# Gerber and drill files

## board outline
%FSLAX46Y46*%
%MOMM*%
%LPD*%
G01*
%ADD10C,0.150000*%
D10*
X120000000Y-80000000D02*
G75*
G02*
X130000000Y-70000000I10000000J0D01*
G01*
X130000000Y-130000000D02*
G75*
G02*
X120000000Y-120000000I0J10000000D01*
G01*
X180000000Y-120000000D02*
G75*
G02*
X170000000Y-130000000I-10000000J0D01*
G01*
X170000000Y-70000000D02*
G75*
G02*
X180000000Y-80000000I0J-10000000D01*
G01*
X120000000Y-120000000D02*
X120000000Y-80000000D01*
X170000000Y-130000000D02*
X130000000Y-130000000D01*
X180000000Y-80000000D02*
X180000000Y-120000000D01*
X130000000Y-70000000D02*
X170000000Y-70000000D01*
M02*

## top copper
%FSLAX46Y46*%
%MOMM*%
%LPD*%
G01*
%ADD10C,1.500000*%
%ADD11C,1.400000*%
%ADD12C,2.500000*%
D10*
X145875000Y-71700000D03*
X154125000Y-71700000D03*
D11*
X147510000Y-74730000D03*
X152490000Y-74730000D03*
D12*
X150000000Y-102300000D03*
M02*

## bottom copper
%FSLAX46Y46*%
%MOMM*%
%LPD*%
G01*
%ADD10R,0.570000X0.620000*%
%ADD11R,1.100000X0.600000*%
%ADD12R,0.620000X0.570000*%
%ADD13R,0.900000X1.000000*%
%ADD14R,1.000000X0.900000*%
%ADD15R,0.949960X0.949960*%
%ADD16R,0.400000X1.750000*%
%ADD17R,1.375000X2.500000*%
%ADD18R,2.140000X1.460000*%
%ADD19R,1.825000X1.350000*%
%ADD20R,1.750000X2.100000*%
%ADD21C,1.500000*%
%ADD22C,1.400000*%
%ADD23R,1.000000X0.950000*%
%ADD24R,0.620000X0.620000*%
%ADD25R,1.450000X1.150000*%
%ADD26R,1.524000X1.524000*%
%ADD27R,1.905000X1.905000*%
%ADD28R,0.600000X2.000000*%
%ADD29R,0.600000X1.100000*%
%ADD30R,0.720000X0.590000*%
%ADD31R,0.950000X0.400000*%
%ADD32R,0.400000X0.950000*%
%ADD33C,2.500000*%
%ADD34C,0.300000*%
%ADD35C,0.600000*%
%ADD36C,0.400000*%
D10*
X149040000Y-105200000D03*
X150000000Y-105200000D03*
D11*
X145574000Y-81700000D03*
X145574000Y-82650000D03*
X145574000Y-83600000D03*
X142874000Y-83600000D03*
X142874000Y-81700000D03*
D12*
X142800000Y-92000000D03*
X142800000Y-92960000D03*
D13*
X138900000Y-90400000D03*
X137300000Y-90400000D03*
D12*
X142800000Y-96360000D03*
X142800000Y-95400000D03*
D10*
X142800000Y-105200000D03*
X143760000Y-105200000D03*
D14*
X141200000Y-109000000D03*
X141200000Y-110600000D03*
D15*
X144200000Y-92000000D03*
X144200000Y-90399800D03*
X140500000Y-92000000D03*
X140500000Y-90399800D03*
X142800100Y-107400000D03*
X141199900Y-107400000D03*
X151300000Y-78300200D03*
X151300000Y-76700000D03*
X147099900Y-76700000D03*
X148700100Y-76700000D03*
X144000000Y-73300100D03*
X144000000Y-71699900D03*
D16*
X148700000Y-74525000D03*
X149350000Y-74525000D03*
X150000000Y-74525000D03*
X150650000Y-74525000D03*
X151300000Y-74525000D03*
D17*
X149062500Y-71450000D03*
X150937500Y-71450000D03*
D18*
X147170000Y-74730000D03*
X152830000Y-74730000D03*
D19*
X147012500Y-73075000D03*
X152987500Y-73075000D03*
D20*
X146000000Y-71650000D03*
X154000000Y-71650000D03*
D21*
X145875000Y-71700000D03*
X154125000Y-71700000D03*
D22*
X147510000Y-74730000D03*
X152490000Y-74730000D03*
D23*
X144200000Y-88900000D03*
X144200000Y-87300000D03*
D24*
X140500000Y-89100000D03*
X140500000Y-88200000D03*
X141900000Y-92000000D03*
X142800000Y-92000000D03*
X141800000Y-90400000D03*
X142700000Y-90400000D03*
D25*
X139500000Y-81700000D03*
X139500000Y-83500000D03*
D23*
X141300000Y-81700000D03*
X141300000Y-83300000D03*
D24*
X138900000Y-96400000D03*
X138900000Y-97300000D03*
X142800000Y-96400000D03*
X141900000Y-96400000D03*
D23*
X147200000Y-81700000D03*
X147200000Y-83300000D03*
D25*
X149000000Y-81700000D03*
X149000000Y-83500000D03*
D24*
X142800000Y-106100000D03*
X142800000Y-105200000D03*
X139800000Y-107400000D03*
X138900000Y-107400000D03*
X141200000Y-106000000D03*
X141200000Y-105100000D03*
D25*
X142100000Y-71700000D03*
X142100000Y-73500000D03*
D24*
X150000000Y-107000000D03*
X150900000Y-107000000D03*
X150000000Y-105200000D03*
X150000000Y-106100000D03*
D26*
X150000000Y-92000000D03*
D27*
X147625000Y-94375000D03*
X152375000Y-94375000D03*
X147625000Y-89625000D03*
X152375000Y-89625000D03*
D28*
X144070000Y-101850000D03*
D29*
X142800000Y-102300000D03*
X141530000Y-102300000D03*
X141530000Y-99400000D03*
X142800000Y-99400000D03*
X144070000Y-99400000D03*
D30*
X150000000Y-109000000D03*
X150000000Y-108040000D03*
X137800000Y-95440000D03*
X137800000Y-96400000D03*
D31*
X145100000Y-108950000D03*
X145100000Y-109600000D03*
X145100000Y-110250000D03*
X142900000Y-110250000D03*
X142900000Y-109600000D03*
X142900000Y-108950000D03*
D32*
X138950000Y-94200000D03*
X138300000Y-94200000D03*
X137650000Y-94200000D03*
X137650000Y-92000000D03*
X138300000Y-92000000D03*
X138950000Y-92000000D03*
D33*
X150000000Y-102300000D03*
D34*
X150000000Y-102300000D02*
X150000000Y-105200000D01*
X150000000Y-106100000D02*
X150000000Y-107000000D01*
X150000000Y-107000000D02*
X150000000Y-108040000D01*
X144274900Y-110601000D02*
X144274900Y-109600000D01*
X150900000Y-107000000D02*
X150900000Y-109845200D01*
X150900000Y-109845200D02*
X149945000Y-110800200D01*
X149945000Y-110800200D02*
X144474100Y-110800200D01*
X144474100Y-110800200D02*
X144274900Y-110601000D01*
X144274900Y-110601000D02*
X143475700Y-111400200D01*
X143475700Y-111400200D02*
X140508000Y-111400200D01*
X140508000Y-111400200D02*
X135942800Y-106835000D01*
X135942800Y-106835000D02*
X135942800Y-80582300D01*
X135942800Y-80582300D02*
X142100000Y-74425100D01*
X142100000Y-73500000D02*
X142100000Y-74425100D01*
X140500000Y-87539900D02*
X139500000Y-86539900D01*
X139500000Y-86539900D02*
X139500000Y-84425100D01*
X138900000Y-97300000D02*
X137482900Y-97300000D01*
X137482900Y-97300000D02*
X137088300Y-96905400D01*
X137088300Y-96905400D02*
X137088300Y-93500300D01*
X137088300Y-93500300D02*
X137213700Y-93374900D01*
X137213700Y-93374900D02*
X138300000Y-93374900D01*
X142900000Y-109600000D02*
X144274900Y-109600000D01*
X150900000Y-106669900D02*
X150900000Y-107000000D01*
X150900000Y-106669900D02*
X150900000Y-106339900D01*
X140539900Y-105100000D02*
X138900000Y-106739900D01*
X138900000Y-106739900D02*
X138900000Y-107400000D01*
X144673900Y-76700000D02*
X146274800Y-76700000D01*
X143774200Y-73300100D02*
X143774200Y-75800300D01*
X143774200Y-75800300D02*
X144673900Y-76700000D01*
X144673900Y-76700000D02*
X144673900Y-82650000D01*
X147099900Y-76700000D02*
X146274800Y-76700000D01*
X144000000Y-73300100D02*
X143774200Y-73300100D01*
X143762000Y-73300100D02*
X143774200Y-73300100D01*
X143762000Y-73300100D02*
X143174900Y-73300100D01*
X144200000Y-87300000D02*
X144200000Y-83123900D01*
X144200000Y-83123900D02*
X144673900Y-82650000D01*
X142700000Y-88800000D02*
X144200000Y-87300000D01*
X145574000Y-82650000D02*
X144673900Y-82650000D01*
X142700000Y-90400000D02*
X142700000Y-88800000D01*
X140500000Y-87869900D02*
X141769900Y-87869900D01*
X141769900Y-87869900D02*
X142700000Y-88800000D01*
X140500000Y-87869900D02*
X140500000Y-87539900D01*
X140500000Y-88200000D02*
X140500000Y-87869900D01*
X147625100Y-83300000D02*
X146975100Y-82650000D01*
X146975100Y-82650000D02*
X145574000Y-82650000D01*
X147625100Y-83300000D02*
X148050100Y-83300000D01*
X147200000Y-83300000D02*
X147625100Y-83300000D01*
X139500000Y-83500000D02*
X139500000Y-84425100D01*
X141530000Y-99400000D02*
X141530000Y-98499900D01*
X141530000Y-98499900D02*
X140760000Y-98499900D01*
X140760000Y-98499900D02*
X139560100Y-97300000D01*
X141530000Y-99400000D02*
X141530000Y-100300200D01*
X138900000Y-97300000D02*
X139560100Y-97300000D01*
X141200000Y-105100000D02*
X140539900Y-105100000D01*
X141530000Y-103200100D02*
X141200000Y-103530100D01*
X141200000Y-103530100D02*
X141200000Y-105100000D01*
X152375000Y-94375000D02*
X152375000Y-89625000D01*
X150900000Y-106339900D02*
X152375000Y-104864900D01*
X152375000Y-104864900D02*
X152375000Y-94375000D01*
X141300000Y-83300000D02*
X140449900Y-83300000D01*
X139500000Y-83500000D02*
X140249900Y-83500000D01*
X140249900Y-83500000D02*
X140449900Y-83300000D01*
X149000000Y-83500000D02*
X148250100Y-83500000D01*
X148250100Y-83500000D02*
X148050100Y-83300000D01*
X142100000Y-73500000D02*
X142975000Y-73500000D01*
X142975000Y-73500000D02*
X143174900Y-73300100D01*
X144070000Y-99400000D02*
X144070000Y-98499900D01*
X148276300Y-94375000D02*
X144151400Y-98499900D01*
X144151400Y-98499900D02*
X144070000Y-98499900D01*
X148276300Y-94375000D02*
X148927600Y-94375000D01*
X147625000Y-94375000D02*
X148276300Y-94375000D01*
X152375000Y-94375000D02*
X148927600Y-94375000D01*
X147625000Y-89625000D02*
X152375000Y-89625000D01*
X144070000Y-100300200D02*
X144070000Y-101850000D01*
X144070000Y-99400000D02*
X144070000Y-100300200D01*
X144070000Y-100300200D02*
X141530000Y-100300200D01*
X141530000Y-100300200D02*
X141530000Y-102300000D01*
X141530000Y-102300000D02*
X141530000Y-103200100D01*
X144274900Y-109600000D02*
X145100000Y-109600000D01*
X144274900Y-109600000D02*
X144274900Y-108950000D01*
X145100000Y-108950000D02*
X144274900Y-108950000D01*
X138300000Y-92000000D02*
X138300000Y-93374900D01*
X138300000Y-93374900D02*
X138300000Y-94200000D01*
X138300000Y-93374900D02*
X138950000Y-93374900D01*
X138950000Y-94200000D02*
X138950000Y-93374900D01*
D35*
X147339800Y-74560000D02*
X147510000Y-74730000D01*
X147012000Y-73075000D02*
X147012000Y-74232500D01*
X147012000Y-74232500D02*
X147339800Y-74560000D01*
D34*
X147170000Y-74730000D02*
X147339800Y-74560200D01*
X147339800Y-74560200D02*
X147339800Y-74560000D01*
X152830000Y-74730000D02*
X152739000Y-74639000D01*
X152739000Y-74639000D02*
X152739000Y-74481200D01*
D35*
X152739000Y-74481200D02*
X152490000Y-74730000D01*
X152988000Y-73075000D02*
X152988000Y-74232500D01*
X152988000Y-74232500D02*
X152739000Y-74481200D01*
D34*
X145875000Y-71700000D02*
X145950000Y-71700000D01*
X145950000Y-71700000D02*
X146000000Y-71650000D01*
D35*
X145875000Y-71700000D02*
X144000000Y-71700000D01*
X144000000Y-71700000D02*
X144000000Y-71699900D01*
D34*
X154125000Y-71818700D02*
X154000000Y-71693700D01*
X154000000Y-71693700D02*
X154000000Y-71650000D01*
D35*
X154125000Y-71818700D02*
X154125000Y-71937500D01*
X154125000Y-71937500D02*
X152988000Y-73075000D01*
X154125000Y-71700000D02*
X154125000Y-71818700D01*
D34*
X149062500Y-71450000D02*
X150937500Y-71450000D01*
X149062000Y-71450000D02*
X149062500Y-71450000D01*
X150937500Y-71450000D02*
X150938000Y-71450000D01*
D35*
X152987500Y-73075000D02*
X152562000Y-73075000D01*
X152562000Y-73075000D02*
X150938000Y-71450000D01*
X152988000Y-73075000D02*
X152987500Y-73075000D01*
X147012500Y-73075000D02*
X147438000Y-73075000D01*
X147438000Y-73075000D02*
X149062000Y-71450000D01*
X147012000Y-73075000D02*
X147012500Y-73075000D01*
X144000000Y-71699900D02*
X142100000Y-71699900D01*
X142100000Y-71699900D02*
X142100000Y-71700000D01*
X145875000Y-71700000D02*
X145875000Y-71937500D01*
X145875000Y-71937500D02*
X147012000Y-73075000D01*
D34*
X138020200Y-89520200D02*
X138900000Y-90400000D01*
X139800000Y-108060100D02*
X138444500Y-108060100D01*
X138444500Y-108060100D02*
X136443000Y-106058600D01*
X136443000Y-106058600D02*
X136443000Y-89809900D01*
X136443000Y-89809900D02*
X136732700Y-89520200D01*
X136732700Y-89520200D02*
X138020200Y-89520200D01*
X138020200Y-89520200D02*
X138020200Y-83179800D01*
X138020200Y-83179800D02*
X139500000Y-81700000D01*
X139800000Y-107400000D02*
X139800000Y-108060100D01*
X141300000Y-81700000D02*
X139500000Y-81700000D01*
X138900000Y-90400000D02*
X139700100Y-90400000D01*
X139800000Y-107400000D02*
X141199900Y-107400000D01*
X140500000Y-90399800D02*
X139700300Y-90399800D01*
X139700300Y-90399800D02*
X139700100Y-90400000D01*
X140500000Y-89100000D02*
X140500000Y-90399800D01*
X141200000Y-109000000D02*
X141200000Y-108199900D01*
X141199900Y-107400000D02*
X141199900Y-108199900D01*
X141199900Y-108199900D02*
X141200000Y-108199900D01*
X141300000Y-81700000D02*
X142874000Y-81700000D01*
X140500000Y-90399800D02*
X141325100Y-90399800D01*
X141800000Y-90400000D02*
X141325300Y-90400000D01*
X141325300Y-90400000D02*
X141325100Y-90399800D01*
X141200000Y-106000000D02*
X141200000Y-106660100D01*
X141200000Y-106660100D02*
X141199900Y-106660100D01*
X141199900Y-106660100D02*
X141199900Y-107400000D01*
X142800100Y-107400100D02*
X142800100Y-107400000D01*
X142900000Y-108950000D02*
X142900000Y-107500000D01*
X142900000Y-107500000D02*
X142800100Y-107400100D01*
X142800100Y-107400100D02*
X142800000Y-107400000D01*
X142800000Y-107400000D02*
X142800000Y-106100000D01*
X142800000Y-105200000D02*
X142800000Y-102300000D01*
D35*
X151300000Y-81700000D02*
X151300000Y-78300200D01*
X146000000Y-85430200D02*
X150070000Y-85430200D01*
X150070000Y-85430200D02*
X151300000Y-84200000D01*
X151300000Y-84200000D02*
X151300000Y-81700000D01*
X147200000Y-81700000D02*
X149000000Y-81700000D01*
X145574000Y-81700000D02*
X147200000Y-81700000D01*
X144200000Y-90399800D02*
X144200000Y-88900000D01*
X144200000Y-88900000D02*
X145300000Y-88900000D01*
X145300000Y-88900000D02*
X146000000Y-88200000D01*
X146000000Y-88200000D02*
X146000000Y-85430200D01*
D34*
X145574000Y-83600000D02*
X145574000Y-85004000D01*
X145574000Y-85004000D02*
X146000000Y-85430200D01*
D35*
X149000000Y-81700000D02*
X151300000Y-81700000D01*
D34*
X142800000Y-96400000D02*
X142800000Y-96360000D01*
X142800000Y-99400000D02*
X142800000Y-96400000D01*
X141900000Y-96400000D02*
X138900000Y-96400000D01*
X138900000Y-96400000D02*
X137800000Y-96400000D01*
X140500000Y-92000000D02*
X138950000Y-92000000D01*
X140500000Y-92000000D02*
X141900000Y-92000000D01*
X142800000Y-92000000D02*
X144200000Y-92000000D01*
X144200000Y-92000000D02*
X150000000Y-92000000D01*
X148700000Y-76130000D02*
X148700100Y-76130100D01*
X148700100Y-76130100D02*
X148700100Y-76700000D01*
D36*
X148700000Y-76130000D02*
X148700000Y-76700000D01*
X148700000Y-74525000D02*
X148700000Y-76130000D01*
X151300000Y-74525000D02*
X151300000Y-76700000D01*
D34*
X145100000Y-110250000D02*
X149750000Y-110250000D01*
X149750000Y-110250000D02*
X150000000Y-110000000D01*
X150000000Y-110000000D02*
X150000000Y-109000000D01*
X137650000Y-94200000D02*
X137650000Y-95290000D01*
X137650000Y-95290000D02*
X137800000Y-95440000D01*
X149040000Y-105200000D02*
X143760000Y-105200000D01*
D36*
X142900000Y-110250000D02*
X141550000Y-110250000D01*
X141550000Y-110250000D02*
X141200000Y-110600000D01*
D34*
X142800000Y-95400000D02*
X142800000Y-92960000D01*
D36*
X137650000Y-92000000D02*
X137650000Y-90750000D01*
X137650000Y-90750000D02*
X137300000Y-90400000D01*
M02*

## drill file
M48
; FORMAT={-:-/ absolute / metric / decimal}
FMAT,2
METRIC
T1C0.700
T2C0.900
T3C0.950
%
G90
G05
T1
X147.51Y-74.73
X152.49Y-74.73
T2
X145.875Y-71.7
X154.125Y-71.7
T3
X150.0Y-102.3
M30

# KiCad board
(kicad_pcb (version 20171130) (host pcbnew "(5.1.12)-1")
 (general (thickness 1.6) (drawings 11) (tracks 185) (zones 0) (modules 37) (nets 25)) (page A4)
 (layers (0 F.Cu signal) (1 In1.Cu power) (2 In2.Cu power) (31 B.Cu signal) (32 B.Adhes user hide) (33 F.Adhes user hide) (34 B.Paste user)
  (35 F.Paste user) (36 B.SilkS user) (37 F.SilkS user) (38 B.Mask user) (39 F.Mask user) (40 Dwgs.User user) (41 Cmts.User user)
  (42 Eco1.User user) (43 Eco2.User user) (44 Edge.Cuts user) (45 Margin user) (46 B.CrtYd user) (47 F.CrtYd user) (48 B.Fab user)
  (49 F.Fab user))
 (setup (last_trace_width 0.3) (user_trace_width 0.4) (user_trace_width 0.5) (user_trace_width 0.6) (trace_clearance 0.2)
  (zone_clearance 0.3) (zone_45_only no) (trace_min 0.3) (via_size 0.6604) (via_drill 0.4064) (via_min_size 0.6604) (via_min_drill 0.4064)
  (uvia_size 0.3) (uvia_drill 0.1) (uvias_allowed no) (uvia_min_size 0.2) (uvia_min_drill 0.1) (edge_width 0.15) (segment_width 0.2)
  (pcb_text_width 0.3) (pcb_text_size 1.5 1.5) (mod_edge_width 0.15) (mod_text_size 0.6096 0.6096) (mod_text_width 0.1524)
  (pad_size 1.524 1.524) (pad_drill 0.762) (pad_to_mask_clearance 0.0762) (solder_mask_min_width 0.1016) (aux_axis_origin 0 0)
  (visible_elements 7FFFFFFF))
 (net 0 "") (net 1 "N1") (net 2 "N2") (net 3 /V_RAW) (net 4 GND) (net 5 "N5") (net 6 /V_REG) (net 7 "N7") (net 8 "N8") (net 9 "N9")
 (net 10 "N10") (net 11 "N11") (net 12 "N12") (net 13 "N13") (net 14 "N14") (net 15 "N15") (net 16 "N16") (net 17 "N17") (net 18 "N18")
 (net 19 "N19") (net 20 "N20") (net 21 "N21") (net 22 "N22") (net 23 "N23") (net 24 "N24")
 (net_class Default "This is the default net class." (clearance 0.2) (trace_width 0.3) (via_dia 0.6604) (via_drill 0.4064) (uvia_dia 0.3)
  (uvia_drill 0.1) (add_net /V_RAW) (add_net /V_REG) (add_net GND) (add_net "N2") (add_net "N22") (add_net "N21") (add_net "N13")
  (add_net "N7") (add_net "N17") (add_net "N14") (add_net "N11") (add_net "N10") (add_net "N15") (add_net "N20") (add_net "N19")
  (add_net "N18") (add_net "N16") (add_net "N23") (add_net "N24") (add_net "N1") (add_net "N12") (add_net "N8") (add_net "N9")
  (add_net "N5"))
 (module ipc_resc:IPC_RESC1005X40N (layer B.Cu) (at 149.52 105.2)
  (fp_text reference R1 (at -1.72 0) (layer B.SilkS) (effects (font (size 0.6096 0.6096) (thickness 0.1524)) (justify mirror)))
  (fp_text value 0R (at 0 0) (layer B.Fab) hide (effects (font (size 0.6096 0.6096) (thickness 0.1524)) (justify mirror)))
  (pad 1 smd rect (at -0.48 0) (size 0.57 0.62) (layers B.Cu B.Paste B.Mask) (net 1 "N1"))
  (pad 2 smd rect (at 0.48 0) (size 0.57 0.62) (layers B.Cu B.Paste B.Mask) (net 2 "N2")))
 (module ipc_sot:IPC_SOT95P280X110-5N (layer B.Cu) (at 144.224 82.65 180)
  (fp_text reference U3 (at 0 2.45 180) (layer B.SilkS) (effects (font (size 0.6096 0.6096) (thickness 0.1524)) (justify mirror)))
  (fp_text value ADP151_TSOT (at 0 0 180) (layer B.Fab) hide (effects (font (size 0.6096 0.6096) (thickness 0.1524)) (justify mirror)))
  (pad 1 smd rect (at -1.35 0.95 180) (size 1.1 0.6) (layers B.Cu B.Paste B.Mask) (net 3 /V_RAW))
  (pad 2 smd rect (at -1.35 0 180) (size 1.1 0.6) (layers B.Cu B.Paste B.Mask) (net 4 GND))
  (pad 3 smd rect (at -1.35 -0.95 180) (size 1.1 0.6) (layers B.Cu B.Paste B.Mask) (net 3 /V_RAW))
  (pad 4 smd rect (at 1.35 -0.95 180) (size 1.1 0.6) (layers B.Cu B.Paste B.Mask) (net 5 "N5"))
  (pad 5 smd rect (at 1.35 0.95 180) (size 1.1 0.6) (layers B.Cu B.Paste B.Mask) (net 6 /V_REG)))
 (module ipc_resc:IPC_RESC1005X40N (layer B.Cu) (at 142.8 92.48 270)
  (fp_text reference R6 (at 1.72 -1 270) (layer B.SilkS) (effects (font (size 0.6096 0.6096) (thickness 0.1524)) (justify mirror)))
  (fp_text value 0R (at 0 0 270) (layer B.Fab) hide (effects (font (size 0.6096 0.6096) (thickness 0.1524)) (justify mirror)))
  (pad 1 smd rect (at -0.48 0 270) (size 0.57 0.62) (layers B.Cu B.Paste B.Mask) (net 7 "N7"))
  (pad 2 smd rect (at 0.48 0 270) (size 0.57 0.62) (layers B.Cu B.Paste B.Mask) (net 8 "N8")))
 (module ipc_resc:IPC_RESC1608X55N (layer B.Cu) (at 138.1 90.4 180)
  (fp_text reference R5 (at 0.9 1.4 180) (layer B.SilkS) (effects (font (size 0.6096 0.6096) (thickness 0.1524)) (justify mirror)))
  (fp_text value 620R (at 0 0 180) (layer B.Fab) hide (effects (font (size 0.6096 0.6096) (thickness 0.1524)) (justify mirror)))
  (pad 1 smd rect (at -0.8 0 180) (size 0.9 1) (layers B.Cu B.Paste B.Mask) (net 6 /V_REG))
  (pad 2 smd rect (at 0.8 0 180) (size 0.9 1) (layers B.Cu B.Paste B.Mask) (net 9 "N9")))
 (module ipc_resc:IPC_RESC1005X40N (layer B.Cu) (at 142.8 95.88 90)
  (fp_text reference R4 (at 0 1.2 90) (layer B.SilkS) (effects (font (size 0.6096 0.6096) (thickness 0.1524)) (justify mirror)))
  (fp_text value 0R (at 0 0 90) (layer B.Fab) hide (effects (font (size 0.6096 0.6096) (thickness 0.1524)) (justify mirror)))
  (pad 1 smd rect (at -0.48 0 90) (size 0.57 0.62) (layers B.Cu B.Paste B.Mask) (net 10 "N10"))
  (pad 2 smd rect (at 0.48 0 90) (size 0.57 0.62) (layers B.Cu B.Paste B.Mask) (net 8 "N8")))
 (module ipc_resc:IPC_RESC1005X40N (layer B.Cu) (at 143.28 105.2)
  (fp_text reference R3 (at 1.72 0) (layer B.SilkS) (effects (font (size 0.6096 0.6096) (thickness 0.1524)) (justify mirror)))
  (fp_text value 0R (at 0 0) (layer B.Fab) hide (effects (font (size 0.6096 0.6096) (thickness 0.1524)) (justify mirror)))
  (pad 1 smd rect (at -0.48 0) (size 0.57 0.62) (layers B.Cu B.Paste B.Mask) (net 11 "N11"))
  (pad 2 smd rect (at 0.48 0) (size 0.57 0.62) (layers B.Cu B.Paste B.Mask) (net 1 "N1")))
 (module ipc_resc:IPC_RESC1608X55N (layer B.Cu) (at 141.2 109.8 270)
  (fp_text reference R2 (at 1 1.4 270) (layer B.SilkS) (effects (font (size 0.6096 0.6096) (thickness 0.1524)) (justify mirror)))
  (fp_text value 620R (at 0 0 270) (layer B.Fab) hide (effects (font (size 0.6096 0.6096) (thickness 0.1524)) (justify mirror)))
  (pad 1 smd rect (at -0.8 0 270) (size 0.9 1) (layers B.Cu B.Paste B.Mask) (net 6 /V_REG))
  (pad 2 smd rect (at 0.8 0 270) (size 0.9 1) (layers B.Cu B.Paste B.Mask) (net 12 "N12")))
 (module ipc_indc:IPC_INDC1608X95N (layer B.Cu) (at 144.2 91.1999 90)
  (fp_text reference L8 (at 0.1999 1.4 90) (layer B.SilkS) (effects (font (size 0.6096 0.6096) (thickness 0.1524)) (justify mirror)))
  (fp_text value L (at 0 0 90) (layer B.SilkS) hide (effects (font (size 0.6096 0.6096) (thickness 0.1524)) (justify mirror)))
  (pad 1 smd rect (at -0.8001 0 90) (size 0.94996 0.94996) (layers B.Cu B.Paste B.Mask) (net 7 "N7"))
  (pad 2 smd rect (at 0.8001 0 90) (size 0.94996 0.94996) (layers B.Cu B.Paste B.Mask) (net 3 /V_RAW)))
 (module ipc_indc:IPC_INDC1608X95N (layer B.Cu) (at 140.5 91.1999 90)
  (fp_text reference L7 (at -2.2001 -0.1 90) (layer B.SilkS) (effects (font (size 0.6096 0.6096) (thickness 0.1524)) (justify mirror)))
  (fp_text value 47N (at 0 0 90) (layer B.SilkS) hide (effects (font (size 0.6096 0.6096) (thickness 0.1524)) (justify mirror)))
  (pad 1 smd rect (at -0.8001 0 90) (size 0.94996 0.94996) (layers B.Cu B.Paste B.Mask) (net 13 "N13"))
  (pad 2 smd rect (at 0.8001 0 90) (size 0.94996 0.94996) (layers B.Cu B.Paste B.Mask) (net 6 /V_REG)))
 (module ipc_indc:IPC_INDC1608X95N (layer B.Cu) (at 142 107.4 180)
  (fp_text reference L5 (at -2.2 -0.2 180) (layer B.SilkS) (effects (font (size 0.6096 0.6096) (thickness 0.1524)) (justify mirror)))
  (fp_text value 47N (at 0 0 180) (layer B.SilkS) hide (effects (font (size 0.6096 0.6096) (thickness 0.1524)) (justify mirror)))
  (pad 1 smd rect (at -0.8001 0 180) (size 0.94996 0.94996) (layers B.Cu B.Paste B.Mask) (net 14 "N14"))
  (pad 2 smd rect (at 0.8001 0 180) (size 0.94996 0.94996) (layers B.Cu B.Paste B.Mask) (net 6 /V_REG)))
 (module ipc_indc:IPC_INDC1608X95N (layer B.Cu) (at 151.3 77.5001 90)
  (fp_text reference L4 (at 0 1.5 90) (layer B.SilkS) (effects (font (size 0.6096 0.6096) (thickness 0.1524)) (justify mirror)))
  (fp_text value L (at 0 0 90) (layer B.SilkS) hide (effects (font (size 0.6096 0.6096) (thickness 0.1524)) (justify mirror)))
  (pad 1 smd rect (at -0.8001 0 90) (size 0.94996 0.94996) (layers B.Cu B.Paste B.Mask) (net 3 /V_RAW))
  (pad 2 smd rect (at 0.8001 0 90) (size 0.94996 0.94996) (layers B.Cu B.Paste B.Mask) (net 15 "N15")))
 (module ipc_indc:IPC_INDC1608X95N (layer B.Cu) (at 147.9 76.7)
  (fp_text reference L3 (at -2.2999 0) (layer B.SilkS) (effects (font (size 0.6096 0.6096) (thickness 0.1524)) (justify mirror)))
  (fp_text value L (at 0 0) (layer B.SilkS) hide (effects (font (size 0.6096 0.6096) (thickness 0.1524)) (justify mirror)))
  (pad 1 smd rect (at -0.8001 0) (size 0.94996 0.94996) (layers B.Cu B.Paste B.Mask) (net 4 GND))
  (pad 2 smd rect (at 0.8001 0) (size 0.94996 0.94996) (layers B.Cu B.Paste B.Mask) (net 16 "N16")))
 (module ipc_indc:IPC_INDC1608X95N (layer B.Cu) (at 144 72.5 90)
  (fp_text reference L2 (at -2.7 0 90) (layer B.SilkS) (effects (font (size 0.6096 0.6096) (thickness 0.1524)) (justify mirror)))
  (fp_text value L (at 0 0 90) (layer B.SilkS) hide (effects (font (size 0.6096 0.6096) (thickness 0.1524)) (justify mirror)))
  (pad 1 smd rect (at -0.8001 0 90) (size 0.94996 0.94996) (layers B.Cu B.Paste B.Mask) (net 4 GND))
  (pad 2 smd rect (at 0.8001 0 90) (size 0.94996 0.94996) (layers B.Cu B.Paste B.Mask) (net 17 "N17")))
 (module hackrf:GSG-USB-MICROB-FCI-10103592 (layer B.Cu) (at 150 70 270)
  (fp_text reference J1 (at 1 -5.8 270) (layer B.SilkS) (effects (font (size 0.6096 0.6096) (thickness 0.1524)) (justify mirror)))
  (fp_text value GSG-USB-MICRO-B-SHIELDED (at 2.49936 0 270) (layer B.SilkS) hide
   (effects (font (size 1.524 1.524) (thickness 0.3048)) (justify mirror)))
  (pad 5 smd rect (at 4.525 1.3 270) (size 1.75 0.4) (layers B.Cu B.Paste B.Mask) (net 16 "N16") (solder_mask_margin 0.1016)
   (clearance 0.2032))
  (pad 4 smd rect (at 4.525 0.65 270) (size 1.75 0.4) (layers B.Cu B.Paste B.Mask) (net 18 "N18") (solder_mask_margin 0.1016)
   (clearance 0.2032))
  (pad 3 smd rect (at 4.525 0 270) (size 1.75 0.4) (layers B.Cu B.Paste B.Mask) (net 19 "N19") (solder_mask_margin 0.1016)
   (clearance 0.2032))
  (pad 2 smd rect (at 4.525 -0.65 270) (size 1.75 0.4) (layers B.Cu B.Paste B.Mask) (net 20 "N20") (solder_mask_margin 0.1016)
   (clearance 0.2032))
  (pad 1 smd rect (at 4.525 -1.3 270) (size 1.75 0.4) (layers B.Cu B.Paste B.Mask) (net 15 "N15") (solder_mask_margin 0.1016)
   (clearance 0.2032))
  (pad 0 smd rect (at 1.45 0.9375 270) (size 2.5 1.375) (layers B.Cu B.Paste B.Mask) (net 17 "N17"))
  (pad 0 smd rect (at 1.45 -0.9375 270) (size 2.5 1.375) (layers B.Cu B.Paste B.Mask) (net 17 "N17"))
  (pad 0 smd rect (at 4.73 2.83 270) (size 1.46 2.14) (layers B.Cu B.Paste B.Mask) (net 17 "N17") (solder_paste_margin_ratio -0.05))
  (pad 0 smd rect (at 4.73 -2.83 270) (size 1.46 2.14) (layers B.Cu B.Paste B.Mask) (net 17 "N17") (solder_paste_margin_ratio -0.05))
  (pad 0 smd rect (at 3.075 2.9875 270) (size 1.35 1.825) (layers B.Cu B.Mask) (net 17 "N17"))
  (pad 0 smd rect (at 3.075 -2.9875 270) (size 1.35 1.825) (layers B.Cu B.Mask) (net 17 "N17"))
  (pad 0 smd rect (at 1.65 4 270) (size 2.1 1.75) (layers B.Cu B.Paste B.Mask) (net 17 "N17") (solder_paste_margin_ratio -0.05))
  (pad 0 smd rect (at 1.65 -4 270) (size 2.1 1.75) (layers B.Cu B.Paste B.Mask) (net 17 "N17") (solder_paste_margin_ratio -0.05))
  (pad 0 thru_hole circle (at 1.7 4.125 270) (size 1.5 1.5) (drill 0.9) (layers *.Cu *.Mask) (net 17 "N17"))
  (pad 0 thru_hole circle (at 1.7 -4.125 270) (size 1.5 1.5) (drill 0.9) (layers *.Cu *.Mask) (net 17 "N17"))
  (pad 0 thru_hole circle (at 4.73 2.49 270) (size 1.4 1.4) (drill 0.7) (layers *.Cu *.Mask) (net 17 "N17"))
  (pad 0 thru_hole circle (at 4.73 -2.49 270) (size 1.4 1.4) (drill 0.7) (layers *.Cu *.Mask) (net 17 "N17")))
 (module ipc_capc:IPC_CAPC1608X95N (layer B.Cu) (at 144.2 88.1 90)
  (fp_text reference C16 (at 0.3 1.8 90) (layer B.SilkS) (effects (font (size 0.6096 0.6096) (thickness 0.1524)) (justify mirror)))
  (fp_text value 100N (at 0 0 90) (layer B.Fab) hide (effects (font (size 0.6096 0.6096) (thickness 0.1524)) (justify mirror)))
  (pad 1 smd rect (at -0.8 0 90) (size 0.95 1) (layers B.Cu B.Paste B.Mask) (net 3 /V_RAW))
  (pad 2 smd rect (at 0.8 0 90) (size 0.95 1) (layers B.Cu B.Paste B.Mask) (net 4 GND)))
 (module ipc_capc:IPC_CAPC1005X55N (layer B.Cu) (at 140.5 88.65 90)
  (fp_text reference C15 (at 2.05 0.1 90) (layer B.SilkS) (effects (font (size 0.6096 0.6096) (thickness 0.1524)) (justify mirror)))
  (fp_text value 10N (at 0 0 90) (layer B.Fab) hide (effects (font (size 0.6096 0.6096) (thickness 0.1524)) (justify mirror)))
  (pad 1 smd rect (at -0.45 0 90) (size 0.62 0.62) (layers B.Cu B.Paste B.Mask) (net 6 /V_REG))
  (pad 2 smd rect (at 0.45 0 90) (size 0.62 0.62) (layers B.Cu B.Paste B.Mask) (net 4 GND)))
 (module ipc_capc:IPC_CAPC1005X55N (layer B.Cu) (at 142.35 92)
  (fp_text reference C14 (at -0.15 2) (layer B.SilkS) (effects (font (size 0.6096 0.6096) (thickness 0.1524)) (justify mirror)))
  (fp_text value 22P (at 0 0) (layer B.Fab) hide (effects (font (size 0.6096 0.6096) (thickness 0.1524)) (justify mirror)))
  (pad 1 smd rect (at -0.45 0) (size 0.62 0.62) (layers B.Cu B.Paste B.Mask) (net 13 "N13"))
  (pad 2 smd rect (at 0.45 0) (size 0.62 0.62) (layers B.Cu B.Paste B.Mask) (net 7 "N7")))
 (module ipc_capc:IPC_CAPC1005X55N (layer B.Cu) (at 142.25 90.4)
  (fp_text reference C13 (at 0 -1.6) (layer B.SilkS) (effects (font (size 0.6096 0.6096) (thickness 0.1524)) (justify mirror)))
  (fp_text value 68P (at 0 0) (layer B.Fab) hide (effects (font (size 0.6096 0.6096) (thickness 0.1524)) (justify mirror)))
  (pad 1 smd rect (at -0.45 0) (size 0.62 0.62) (layers B.Cu B.Paste B.Mask) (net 6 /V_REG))
  (pad 2 smd rect (at 0.45 0) (size 0.62 0.62) (layers B.Cu B.Paste B.Mask) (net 4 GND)))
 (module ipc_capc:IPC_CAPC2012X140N (layer B.Cu) (at 139.5 82.6 270)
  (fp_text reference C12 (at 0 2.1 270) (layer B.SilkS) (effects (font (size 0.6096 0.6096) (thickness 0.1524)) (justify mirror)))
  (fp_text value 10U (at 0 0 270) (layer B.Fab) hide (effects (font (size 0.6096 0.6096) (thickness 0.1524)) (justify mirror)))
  (pad 1 smd rect (at -0.9 0 270) (size 1.15 1.45) (layers B.Cu B.Paste B.Mask) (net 6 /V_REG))
  (pad 2 smd rect (at 0.9 0 270) (size 1.15 1.45) (layers B.Cu B.Paste B.Mask) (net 4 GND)))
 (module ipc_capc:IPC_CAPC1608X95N (layer B.Cu) (at 141.3 82.5 270)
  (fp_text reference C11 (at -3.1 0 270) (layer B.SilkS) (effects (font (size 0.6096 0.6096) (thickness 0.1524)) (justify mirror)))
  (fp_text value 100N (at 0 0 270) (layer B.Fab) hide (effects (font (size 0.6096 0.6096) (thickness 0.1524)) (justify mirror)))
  (pad 1 smd rect (at -0.8 0 270) (size 0.95 1) (layers B.Cu B.Paste B.Mask) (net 6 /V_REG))
  (pad 2 smd rect (at 0.8 0 270) (size 0.95 1) (layers B.Cu B.Paste B.Mask) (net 4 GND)))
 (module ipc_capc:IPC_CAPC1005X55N (layer B.Cu) (at 138.9 96.85 270)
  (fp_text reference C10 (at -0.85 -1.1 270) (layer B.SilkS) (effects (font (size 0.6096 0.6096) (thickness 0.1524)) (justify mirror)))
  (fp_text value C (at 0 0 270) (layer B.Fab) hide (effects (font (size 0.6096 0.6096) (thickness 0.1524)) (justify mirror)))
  (pad 1 smd rect (at -0.45 0 270) (size 0.62 0.62) (layers B.Cu B.Paste B.Mask) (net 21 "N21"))
  (pad 2 smd rect (at 0.45 0 270) (size 0.62 0.62) (layers B.Cu B.Paste B.Mask) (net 4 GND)))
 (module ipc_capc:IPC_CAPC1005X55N (layer B.Cu) (at 142.35 96.4 180)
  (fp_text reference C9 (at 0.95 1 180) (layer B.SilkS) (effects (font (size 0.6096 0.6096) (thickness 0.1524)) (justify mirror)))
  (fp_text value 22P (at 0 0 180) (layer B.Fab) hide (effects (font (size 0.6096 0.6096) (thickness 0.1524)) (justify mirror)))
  (pad 1 smd rect (at -0.45 0 180) (size 0.62 0.62) (layers B.Cu B.Paste B.Mask) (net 10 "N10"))
  (pad 2 smd rect (at 0.45 0 180) (size 0.62 0.62) (layers B.Cu B.Paste B.Mask) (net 21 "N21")))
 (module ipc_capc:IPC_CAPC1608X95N (layer B.Cu) (at 147.2 82.5 270)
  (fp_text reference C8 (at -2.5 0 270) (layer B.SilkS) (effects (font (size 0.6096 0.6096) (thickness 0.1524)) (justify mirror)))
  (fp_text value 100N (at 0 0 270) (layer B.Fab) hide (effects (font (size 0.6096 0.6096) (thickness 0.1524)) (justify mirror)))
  (pad 1 smd rect (at -0.8 0 270) (size 0.95 1) (layers B.Cu B.Paste B.Mask) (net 3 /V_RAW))
  (pad 2 smd rect (at 0.8 0 270) (size 0.95 1) (layers B.Cu B.Paste B.Mask) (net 4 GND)))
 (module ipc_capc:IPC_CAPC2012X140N (layer B.Cu) (at 149 82.6 270)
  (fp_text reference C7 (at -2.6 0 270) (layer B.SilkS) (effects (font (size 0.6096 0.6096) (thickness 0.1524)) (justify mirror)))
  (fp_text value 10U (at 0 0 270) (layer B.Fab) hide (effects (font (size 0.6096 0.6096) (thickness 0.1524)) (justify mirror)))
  (pad 1 smd rect (at -0.9 0 270) (size 1.15 1.45) (layers B.Cu B.Paste B.Mask) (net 3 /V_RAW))
  (pad 2 smd rect (at 0.9 0 270) (size 1.15 1.45) (layers B.Cu B.Paste B.Mask) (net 4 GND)))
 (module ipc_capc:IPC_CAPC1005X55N (layer B.Cu) (at 142.8 105.65 90)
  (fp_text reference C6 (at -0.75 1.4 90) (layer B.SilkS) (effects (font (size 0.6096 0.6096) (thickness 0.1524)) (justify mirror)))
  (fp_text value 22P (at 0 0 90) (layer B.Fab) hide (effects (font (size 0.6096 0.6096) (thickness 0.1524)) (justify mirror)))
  (pad 1 smd rect (at -0.45 0 90) (size 0.62 0.62) (layers B.Cu B.Paste B.Mask) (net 14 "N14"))
  (pad 2 smd rect (at 0.45 0 90) (size 0.62 0.62) (layers B.Cu B.Paste B.Mask) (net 11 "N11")))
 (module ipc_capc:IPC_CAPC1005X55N (layer B.Cu) (at 139.35 107.4 180)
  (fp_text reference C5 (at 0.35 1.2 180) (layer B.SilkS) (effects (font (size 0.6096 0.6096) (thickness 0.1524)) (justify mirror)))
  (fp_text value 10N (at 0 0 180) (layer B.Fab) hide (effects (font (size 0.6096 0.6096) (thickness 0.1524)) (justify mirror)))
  (pad 1 smd rect (at -0.45 0 180) (size 0.62 0.62) (layers B.Cu B.Paste B.Mask) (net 6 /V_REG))
  (pad 2 smd rect (at 0.45 0 180) (size 0.62 0.62) (layers B.Cu B.Paste B.Mask) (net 4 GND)))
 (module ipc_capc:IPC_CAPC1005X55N (layer B.Cu) (at 141.2 105.55 90)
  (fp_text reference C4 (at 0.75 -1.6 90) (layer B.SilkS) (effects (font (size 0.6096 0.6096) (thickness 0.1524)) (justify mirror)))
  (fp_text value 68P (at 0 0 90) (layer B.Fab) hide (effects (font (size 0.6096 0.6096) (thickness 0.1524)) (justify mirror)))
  (pad 1 smd rect (at -0.45 0 90) (size 0.62 0.62) (layers B.Cu B.Paste B.Mask) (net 6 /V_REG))
  (pad 2 smd rect (at 0.45 0 90) (size 0.62 0.62) (layers B.Cu B.Paste B.Mask) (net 4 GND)))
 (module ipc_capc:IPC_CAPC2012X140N (layer B.Cu) (at 142.1 72.6 270)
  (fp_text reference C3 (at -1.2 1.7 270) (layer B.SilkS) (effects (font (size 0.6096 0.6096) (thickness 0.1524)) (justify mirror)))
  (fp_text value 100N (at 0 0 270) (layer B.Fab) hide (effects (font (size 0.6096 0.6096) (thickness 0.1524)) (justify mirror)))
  (pad 1 smd rect (at -0.9 0 270) (size 1.15 1.45) (layers B.Cu B.Paste B.Mask) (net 17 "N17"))
  (pad 2 smd rect (at 0.9 0 270) (size 1.15 1.45) (layers B.Cu B.Paste B.Mask) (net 4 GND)))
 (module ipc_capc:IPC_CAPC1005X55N (layer B.Cu) (at 150.45 107)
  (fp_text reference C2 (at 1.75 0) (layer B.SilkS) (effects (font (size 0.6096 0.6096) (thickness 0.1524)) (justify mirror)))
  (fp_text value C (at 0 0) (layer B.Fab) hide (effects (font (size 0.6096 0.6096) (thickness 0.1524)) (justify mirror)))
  (pad 1 smd rect (at -0.45 0) (size 0.62 0.62) (layers B.Cu B.Paste B.Mask) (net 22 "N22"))
  (pad 2 smd rect (at 0.45 0) (size 0.62 0.62) (layers B.Cu B.Paste B.Mask) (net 4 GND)))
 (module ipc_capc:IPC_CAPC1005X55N (layer B.Cu) (at 150 105.65 270)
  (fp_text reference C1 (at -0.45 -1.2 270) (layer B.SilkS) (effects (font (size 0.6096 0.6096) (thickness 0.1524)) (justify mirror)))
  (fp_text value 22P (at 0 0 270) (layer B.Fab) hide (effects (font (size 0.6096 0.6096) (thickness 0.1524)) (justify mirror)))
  (pad 1 smd rect (at -0.45 0 270) (size 0.62 0.62) (layers B.Cu B.Paste B.Mask) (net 2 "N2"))
  (pad 2 smd rect (at 0.45 0 270) (size 0.62 0.62) (layers B.Cu B.Paste B.Mask) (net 22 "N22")))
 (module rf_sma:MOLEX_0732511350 (layer B.Cu) (at 150 92)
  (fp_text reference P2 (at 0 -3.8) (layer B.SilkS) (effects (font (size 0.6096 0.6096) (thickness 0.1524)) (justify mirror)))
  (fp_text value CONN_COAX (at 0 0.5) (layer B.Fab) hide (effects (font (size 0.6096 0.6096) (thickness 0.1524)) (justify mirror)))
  (pad 1 smd rect (at 0 0) (size 1.524 1.524) (layers B.Cu B.Paste B.Mask) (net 7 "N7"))
  (pad 2 smd rect (at -2.375 2.375) (size 1.905 1.905) (layers B.Cu B.Paste B.Mask) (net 4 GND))
  (pad 2 smd rect (at 2.375 2.375) (size 1.905 1.905) (layers B.Cu B.Paste B.Mask) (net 4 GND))
  (pad 2 smd rect (at -2.375 -2.375) (size 1.905 1.905) (layers B.Cu B.Paste B.Mask) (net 4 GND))
  (pad 2 smd rect (at 2.375 -2.375) (size 1.905 1.905) (layers B.Cu B.Paste B.Mask) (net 4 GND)))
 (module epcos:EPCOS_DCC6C (layer B.Cu) (at 142.8 100.85 90)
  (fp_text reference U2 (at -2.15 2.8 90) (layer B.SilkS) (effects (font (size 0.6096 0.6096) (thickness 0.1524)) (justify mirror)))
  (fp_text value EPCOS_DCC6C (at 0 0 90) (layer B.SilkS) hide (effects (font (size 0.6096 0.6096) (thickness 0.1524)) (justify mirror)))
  (pad 1 smd rect (at -1 1.27 90) (size 2 0.6) (layers B.Cu B.Paste B.Mask) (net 4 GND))
  (pad 2 smd rect (at -1.45 0 90) (size 1.1 0.6) (layers B.Cu B.Paste B.Mask) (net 11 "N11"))
  (pad 3 smd rect (at -1.45 -1.27 90) (size 1.1 0.6) (layers B.Cu B.Paste B.Mask) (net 4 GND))
  (pad 4 smd rect (at 1.45 -1.27 90) (size 1.1 0.6) (layers B.Cu B.Paste B.Mask) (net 4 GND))
  (pad 5 smd rect (at 1.45 0 90) (size 1.1 0.6) (layers B.Cu B.Paste B.Mask) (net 10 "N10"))
  (pad 6 smd rect (at 1.45 1.27 90) (size 1.1 0.6) (layers B.Cu B.Paste B.Mask) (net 4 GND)))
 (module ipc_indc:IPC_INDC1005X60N (layer B.Cu) (at 150 108.52 90)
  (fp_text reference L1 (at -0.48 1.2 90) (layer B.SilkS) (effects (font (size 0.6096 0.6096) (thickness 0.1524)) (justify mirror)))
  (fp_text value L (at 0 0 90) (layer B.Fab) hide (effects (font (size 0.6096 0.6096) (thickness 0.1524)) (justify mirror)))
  (pad 1 smd rect (at -0.48 0 90) (size 0.59 0.72) (layers B.Cu B.Paste B.Mask) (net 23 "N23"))
  (pad 2 smd rect (at 0.48 0 90) (size 0.59 0.72) (layers B.Cu B.Paste B.Mask) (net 22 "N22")))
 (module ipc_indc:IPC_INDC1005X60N (layer B.Cu) (at 137.8 95.92 270)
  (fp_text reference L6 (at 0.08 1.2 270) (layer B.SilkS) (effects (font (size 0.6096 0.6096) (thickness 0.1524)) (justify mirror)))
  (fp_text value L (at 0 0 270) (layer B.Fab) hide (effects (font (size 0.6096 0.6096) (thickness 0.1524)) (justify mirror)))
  (pad 1 smd rect (at -0.48 0 270) (size 0.59 0.72) (layers B.Cu B.Paste B.Mask) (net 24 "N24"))
  (pad 2 smd rect (at 0.48 0 270) (size 0.59 0.72) (layers B.Cu B.Paste B.Mask) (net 21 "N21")))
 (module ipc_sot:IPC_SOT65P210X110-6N (layer B.Cu) (at 144 109.6 180)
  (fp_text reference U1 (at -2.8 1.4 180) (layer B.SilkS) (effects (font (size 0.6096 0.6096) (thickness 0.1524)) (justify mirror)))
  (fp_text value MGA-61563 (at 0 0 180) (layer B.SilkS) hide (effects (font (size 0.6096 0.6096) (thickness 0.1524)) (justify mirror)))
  (pad 1 smd rect (at -1.1 0.65 180) (size 0.95 0.4) (layers B.Cu B.Paste B.Mask) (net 4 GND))
  (pad 2 smd rect (at -1.1 0 180) (size 0.95 0.4) (layers B.Cu B.Paste B.Mask) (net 4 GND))
  (pad 3 smd rect (at -1.1 -0.65 180) (size 0.95 0.4) (layers B.Cu B.Paste B.Mask) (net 23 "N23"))
  (pad 4 smd rect (at 1.1 -0.65 180) (size 0.95 0.4) (layers B.Cu B.Paste B.Mask) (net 12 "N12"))
  (pad 5 smd rect (at 1.1 0 180) (size 0.95 0.4) (layers B.Cu B.Paste B.Mask) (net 4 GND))
  (pad 6 smd rect (at 1.1 0.65 180) (size 0.95 0.4) (layers B.Cu B.Paste B.Mask) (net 14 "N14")))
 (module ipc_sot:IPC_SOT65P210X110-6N (layer B.Cu) (at 138.3 93.1 90)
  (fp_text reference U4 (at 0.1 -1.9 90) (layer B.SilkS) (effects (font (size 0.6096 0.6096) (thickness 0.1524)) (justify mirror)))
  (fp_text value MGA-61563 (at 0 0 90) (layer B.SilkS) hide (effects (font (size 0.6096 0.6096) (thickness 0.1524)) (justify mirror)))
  (pad 1 smd rect (at -1.1 0.65 90) (size 0.95 0.4) (layers B.Cu B.Paste B.Mask) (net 4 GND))
  (pad 2 smd rect (at -1.1 0 90) (size 0.95 0.4) (layers B.Cu B.Paste B.Mask) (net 4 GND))
  (pad 3 smd rect (at -1.1 -0.65 90) (size 0.95 0.4) (layers B.Cu B.Paste B.Mask) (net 24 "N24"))
  (pad 4 smd rect (at 1.1 -0.65 90) (size 0.95 0.4) (layers B.Cu B.Paste B.Mask) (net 9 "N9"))
  (pad 5 smd rect (at 1.1 0 90) (size 0.95 0.4) (layers B.Cu B.Paste B.Mask) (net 4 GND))
  (pad 6 smd rect (at 1.1 0.65 90) (size 0.95 0.4) (layers B.Cu B.Paste B.Mask) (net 13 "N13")))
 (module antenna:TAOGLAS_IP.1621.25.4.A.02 (layer F.Cu) (at 150 100)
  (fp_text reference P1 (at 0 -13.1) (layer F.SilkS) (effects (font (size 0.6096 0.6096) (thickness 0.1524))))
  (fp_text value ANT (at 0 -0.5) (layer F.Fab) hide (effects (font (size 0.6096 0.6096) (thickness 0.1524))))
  (pad 1 thru_hole circle (at 0 2.3) (size 2.5 2.5) (drill 0.95) (layers B.Cu) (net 2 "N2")))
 (gr_arc (start 130 80) (end 120 80) (angle 90) (layer Edge.Cuts) (width 0.15))
 (gr_arc (start 130 120) (end 130 130) (angle 90) (layer Edge.Cuts) (width 0.15))
 (gr_arc (start 170 120) (end 180 120) (angle 90) (layer Edge.Cuts) (width 0.15))
 (gr_arc (start 170 80) (end 170 70) (angle 90) (layer Edge.Cuts) (width 0.15))
 (gr_line (start 120 120) (end 120 80) (layer Edge.Cuts) (width 0.15))
 (gr_line (start 170 130) (end 130 130) (layer Edge.Cuts) (width 0.15))
 (gr_line (start 180 80) (end 180 120) (layer Edge.Cuts) (width 0.15))
 (gr_line (start 130 70) (end 170 70) (layer Edge.Cuts) (width 0.15))
 (segment (start 150 102.3) (end 150 105.2) (width 0.3) (layer B.Cu) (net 2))
 (segment (start 150 106.1) (end 150 107) (width 0.3) (layer B.Cu) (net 22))
 (segment (start 150 107) (end 150 108.04) (width 0.3) (layer B.Cu) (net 22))
 (segment (start 144.2749 110.601) (end 144.2749 109.6) (width 0.3) (layer B.Cu) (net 4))
 (segment (start 150.9 107) (end 150.9 109.8452) (width 0.3) (layer B.Cu) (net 4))
 (segment (start 150.9 109.8452) (end 149.945 110.8002) (width 0.3) (layer B.Cu) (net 4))
 (segment (start 149.945 110.8002) (end 144.4741 110.8002) (width 0.3) (layer B.Cu) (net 4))
 (segment (start 144.4741 110.8002) (end 144.2749 110.601) (width 0.3) (layer B.Cu) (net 4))
 (segment (start 144.2749 110.601) (end 143.4757 111.4002) (width 0.3) (layer B.Cu) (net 4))
 (segment (start 143.4757 111.4002) (end 140.508 111.4002) (width 0.3) (layer B.Cu) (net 4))
 (segment (start 140.508 111.4002) (end 135.9428 106.835) (width 0.3) (layer B.Cu) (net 4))
 (segment (start 135.9428 106.835) (end 135.9428 80.5823) (width 0.3) (layer B.Cu) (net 4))
 (segment (start 135.9428 80.5823) (end 142.1 74.4251) (width 0.3) (layer B.Cu) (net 4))
 (segment (start 142.1 73.5) (end 142.1 74.4251) (width 0.3) (layer B.Cu) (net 4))
 (segment (start 140.5 87.5399) (end 139.5 86.5399) (width 0.3) (layer B.Cu) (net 4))
 (segment (start 139.5 86.5399) (end 139.5 84.4251) (width 0.3) (layer B.Cu) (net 4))
 (segment (start 138.9 97.3) (end 137.4829 97.3) (width 0.3) (layer B.Cu) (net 4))
 (segment (start 137.4829 97.3) (end 137.0883 96.9054) (width 0.3) (layer B.Cu) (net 4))
 (segment (start 137.0883 96.9054) (end 137.0883 93.5003) (width 0.3) (layer B.Cu) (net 4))
 (segment (start 137.0883 93.5003) (end 137.2137 93.3749) (width 0.3) (layer B.Cu) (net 4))
 (segment (start 137.2137 93.3749) (end 138.3 93.3749) (width 0.3) (layer B.Cu) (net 4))
 (segment (start 142.9 109.6) (end 144.2749 109.6) (width 0.3) (layer B.Cu) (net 4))
 (segment (start 150.9 106.6699) (end 150.9 107) (width 0.3) (layer B.Cu) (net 4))
 (segment (start 150.9 106.6699) (end 150.9 106.3399) (width 0.3) (layer B.Cu) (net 4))
 (segment (start 140.5399 105.1) (end 138.9 106.7399) (width 0.3) (layer B.Cu) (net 4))
 (segment (start 138.9 106.7399) (end 138.9 107.4) (width 0.3) (layer B.Cu) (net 4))
 (segment (start 144.6739 76.7) (end 146.2748 76.7) (width 0.3) (layer B.Cu) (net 4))
 (segment (start 143.7742 73.3001) (end 143.7742 75.8003) (width 0.3) (layer B.Cu) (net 4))
 (segment (start 143.7742 75.8003) (end 144.6739 76.7) (width 0.3) (layer B.Cu) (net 4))
 (segment (start 144.6739 76.7) (end 144.6739 82.65) (width 0.3) (layer B.Cu) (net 4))
 (segment (start 147.0999 76.7) (end 146.2748 76.7) (width 0.3) (layer B.Cu) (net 4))
 (segment (start 144 73.3001) (end 143.7742 73.3001) (width 0.3) (layer B.Cu) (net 4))
 (segment (start 143.762 73.3001) (end 143.7742 73.3001) (width 0.3) (layer B.Cu) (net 4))
 (segment (start 143.762 73.3001) (end 143.1749 73.3001) (width 0.3) (layer B.Cu) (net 4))
 (segment (start 144.2 87.3) (end 144.2 83.1239) (width 0.3) (layer B.Cu) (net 4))
 (segment (start 144.2 83.1239) (end 144.6739 82.65) (width 0.3) (layer B.Cu) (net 4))
 (segment (start 142.7 88.8) (end 144.2 87.3) (width 0.3) (layer B.Cu) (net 4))
 (segment (start 145.574 82.65) (end 144.6739 82.65) (width 0.3) (layer B.Cu) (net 4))
 (segment (start 142.7 90.4) (end 142.7 88.8) (width 0.3) (layer B.Cu) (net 4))
 (segment (start 140.5 87.8699) (end 141.7699 87.8699) (width 0.3) (layer B.Cu) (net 4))
 (segment (start 141.7699 87.8699) (end 142.7 88.8) (width 0.3) (layer B.Cu) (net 4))
 (segment (start 140.5 87.8699) (end 140.5 87.5399) (width 0.3) (layer B.Cu) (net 4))
 (segment (start 140.5 88.2) (end 140.5 87.8699) (width 0.3) (layer B.Cu) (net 4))
 (segment (start 147.6251 83.3) (end 146.9751 82.65) (width 0.3) (layer B.Cu) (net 4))
 (segment (start 146.9751 82.65) (end 145.574 82.65) (width 0.3) (layer B.Cu) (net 4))
 (segment (start 147.6251 83.3) (end 148.0501 83.3) (width 0.3) (layer B.Cu) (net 4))
 (segment (start 147.2 83.3) (end 147.6251 83.3) (width 0.3) (layer B.Cu) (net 4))
 (segment (start 139.5 83.5) (end 139.5 84.4251) (width 0.3) (layer B.Cu) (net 4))
 (segment (start 141.53 99.4) (end 141.53 98.4999) (width 0.3) (layer B.Cu) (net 4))
 (segment (start 141.53 98.4999) (end 140.76 98.4999) (width 0.3) (layer B.Cu) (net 4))
 (segment (start 140.76 98.4999) (end 139.5601 97.3) (width 0.3) (layer B.Cu) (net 4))
 (segment (start 141.53 99.4) (end 141.53 100.3002) (width 0.3) (layer B.Cu) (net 4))
 (segment (start 138.9 97.3) (end 139.5601 97.3) (width 0.3) (layer B.Cu) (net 4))
 (segment (start 141.2 105.1) (end 140.5399 105.1) (width 0.3) (layer B.Cu) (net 4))
 (segment (start 141.53 103.2001) (end 141.2 103.5301) (width 0.3) (layer B.Cu) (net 4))
 (segment (start 141.2 103.5301) (end 141.2 105.1) (width 0.3) (layer B.Cu) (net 4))
 (segment (start 152.375 94.375) (end 152.375 89.625) (width 0.3) (layer B.Cu) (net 4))
 (segment (start 150.9 106.3399) (end 152.375 104.8649) (width 0.3) (layer B.Cu) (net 4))
 (segment (start 152.375 104.8649) (end 152.375 94.375) (width 0.3) (layer B.Cu) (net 4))
 (segment (start 141.3 83.3) (end 140.4499 83.3) (width 0.3) (layer B.Cu) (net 4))
 (segment (start 139.5 83.5) (end 140.2499 83.5) (width 0.3) (layer B.Cu) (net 4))
 (segment (start 140.2499 83.5) (end 140.4499 83.3) (width 0.3) (layer B.Cu) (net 4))
 (segment (start 149 83.5) (end 148.2501 83.5) (width 0.3) (layer B.Cu) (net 4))
 (segment (start 148.2501 83.5) (end 148.0501 83.3) (width 0.3) (layer B.Cu) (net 4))
 (segment (start 142.1 73.5) (end 142.975 73.5) (width 0.3) (layer B.Cu) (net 4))
 (segment (start 142.975 73.5) (end 143.1749 73.3001) (width 0.3) (layer B.Cu) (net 4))
 (segment (start 144.07 99.4) (end 144.07 98.4999) (width 0.3) (layer B.Cu) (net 4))
 (segment (start 148.2763 94.375) (end 144.1514 98.4999) (width 0.3) (layer B.Cu) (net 4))
 (segment (start 144.1514 98.4999) (end 144.07 98.4999) (width 0.3) (layer B.Cu) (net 4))
 (segment (start 148.2763 94.375) (end 148.9276 94.375) (width 0.3) (layer B.Cu) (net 4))
 (segment (start 147.625 94.375) (end 148.2763 94.375) (width 0.3) (layer B.Cu) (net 4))
 (segment (start 152.375 94.375) (end 148.9276 94.375) (width 0.3) (layer B.Cu) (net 4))
 (segment (start 147.625 89.625) (end 152.375 89.625) (width 0.3) (layer B.Cu) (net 4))
 (segment (start 144.07 100.3002) (end 144.07 101.85) (width 0.3) (layer B.Cu) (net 4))
 (segment (start 144.07 99.4) (end 144.07 100.3002) (width 0.3) (layer B.Cu) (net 4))
 (segment (start 144.07 100.3002) (end 141.53 100.3002) (width 0.3) (layer B.Cu) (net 4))
 (segment (start 141.53 100.3002) (end 141.53 102.3) (width 0.3) (layer B.Cu) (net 4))
 (segment (start 141.53 102.3) (end 141.53 103.2001) (width 0.3) (layer B.Cu) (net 4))
 (segment (start 144.2749 109.6) (end 145.1 109.6) (width 0.3) (layer B.Cu) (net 4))
 (segment (start 144.2749 109.6) (end 144.2749 108.95) (width 0.3) (layer B.Cu) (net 4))
 (segment (start 145.1 108.95) (end 144.2749 108.95) (width 0.3) (layer B.Cu) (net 4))
 (segment (start 138.3 92) (end 138.3 93.3749) (width 0.3) (layer B.Cu) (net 4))
 (segment (start 138.3 93.3749) (end 138.3 94.2) (width 0.3) (layer B.Cu) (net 4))
 (segment (start 138.3 93.3749) (end 138.95 93.3749) (width 0.3) (layer B.Cu) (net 4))
 (segment (start 138.95 94.2) (end 138.95 93.3749) (width 0.3) (layer B.Cu) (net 4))
 (segment (start 147.3398 74.56) (end 147.51 74.73) (width 0.6) (layer B.Cu) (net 17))
 (segment (start 147.012 73.075) (end 147.012 74.2325) (width 0.6) (layer B.Cu) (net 17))
 (segment (start 147.012 74.2325) (end 147.3398 74.56) (width 0.6) (layer B.Cu) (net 17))
 (segment (start 147.17 74.73) (end 147.3398 74.5602) (width 0.3) (layer B.Cu) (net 17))
 (segment (start 147.3398 74.5602) (end 147.3398 74.56) (width 0.3) (layer B.Cu) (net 17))
 (segment (start 152.83 74.73) (end 152.739 74.639) (width 0.3) (layer B.Cu) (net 17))
 (segment (start 152.739 74.639) (end 152.739 74.4812) (width 0.3) (layer B.Cu) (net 17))
 (segment (start 152.739 74.4812) (end 152.49 74.73) (width 0.6) (layer B.Cu) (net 17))
 (segment (start 152.988 73.075) (end 152.988 74.2325) (width 0.6) (layer B.Cu) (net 17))
 (segment (start 152.988 74.2325) (end 152.739 74.4812) (width 0.6) (layer B.Cu) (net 17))
 (segment (start 145.875 71.7) (end 145.95 71.7) (width 0.3) (layer B.Cu) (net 17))
 (segment (start 145.95 71.7) (end 146 71.65) (width 0.3) (layer B.Cu) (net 17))
 (segment (start 145.875 71.7) (end 144 71.7) (width 0.6) (layer B.Cu) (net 17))
 (segment (start 144 71.7) (end 144 71.6999) (width 0.6) (layer B.Cu) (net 17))
 (segment (start 154.125 71.8187) (end 154 71.6937) (width 0.3) (layer B.Cu) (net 17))
 (segment (start 154 71.6937) (end 154 71.65) (width 0.3) (layer B.Cu) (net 17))
 (segment (start 154.125 71.8187) (end 154.125 71.9375) (width 0.6) (layer B.Cu) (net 17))
 (segment (start 154.125 71.9375) (end 152.988 73.075) (width 0.6) (layer B.Cu) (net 17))
 (segment (start 154.125 71.7) (end 154.125 71.8187) (width 0.6) (layer B.Cu) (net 17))
 (segment (start 149.0625 71.45) (end 150.9375 71.45) (width 0.3) (layer B.Cu) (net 17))
 (segment (start 149.062 71.45) (end 149.0625 71.45) (width 0.3) (layer B.Cu) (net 17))
 (segment (start 150.9375 71.45) (end 150.938 71.45) (width 0.3) (layer B.Cu) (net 17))
 (segment (start 152.9875 73.075) (end 152.562 73.075) (width 0.6) (layer B.Cu) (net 17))
 (segment (start 152.562 73.075) (end 150.938 71.45) (width 0.6) (layer B.Cu) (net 17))
 (segment (start 152.988 73.075) (end 152.9875 73.075) (width 0.6) (layer B.Cu) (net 17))
 (segment (start 147.0125 73.075) (end 147.438 73.075) (width 0.6) (layer B.Cu) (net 17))
 (segment (start 147.438 73.075) (end 149.062 71.45) (width 0.6) (layer B.Cu) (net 17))
 (segment (start 147.012 73.075) (end 147.0125 73.075) (width 0.6) (layer B.Cu) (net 17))
 (segment (start 144 71.6999) (end 142.1 71.6999) (width 0.6) (layer B.Cu) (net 17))
 (segment (start 142.1 71.6999) (end 142.1 71.7) (width 0.6) (layer B.Cu) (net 17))
 (segment (start 145.875 71.7) (end 145.875 71.9375) (width 0.6) (layer B.Cu) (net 17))
 (segment (start 145.875 71.9375) (end 147.012 73.075) (width 0.6) (layer B.Cu) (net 17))
 (segment (start 138.0202 89.5202) (end 138.9 90.4) (width 0.3) (layer B.Cu) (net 6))
 (segment (start 139.8 108.0601) (end 138.4445 108.0601) (width 0.3) (layer B.Cu) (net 6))
 (segment (start 138.4445 108.0601) (end 136.443 106.0586) (width 0.3) (layer B.Cu) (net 6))
 (segment (start 136.443 106.0586) (end 136.443 89.8099) (width 0.3) (layer B.Cu) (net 6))
 (segment (start 136.443 89.8099) (end 136.7327 89.5202) (width 0.3) (layer B.Cu) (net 6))
 (segment (start 136.7327 89.5202) (end 138.0202 89.5202) (width 0.3) (layer B.Cu) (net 6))
 (segment (start 138.0202 89.5202) (end 138.0202 83.1798) (width 0.3) (layer B.Cu) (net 6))
 (segment (start 138.0202 83.1798) (end 139.5 81.7) (width 0.3) (layer B.Cu) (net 6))
 (segment (start 139.8 107.4) (end 139.8 108.0601) (width 0.3) (layer B.Cu) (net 6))
 (segment (start 141.3 81.7) (end 139.5 81.7) (width 0.3) (layer B.Cu) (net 6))
 (segment (start 138.9 90.4) (end 139.7001 90.4) (width 0.3) (layer B.Cu) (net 6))
 (segment (start 139.8 107.4) (end 141.1999 107.4) (width 0.3) (layer B.Cu) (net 6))
 (segment (start 140.5 90.3998) (end 139.7003 90.3998) (width 0.3) (layer B.Cu) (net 6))
 (segment (start 139.7003 90.3998) (end 139.7001 90.4) (width 0.3) (layer B.Cu) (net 6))
 (segment (start 140.5 89.1) (end 140.5 90.3998) (width 0.3) (layer B.Cu) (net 6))
 (segment (start 141.2 109) (end 141.2 108.1999) (width 0.3) (layer B.Cu) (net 6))
 (segment (start 141.1999 107.4) (end 141.1999 108.1999) (width 0.3) (layer B.Cu) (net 6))
 (segment (start 141.1999 108.1999) (end 141.2 108.1999) (width 0.3) (layer B.Cu) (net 6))
 (segment (start 141.3 81.7) (end 142.874 81.7) (width 0.3) (layer B.Cu) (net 6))
 (segment (start 140.5 90.3998) (end 141.3251 90.3998) (width 0.3) (layer B.Cu) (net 6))
 (segment (start 141.8 90.4) (end 141.3253 90.4) (width 0.3) (layer B.Cu) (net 6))
 (segment (start 141.3253 90.4) (end 141.3251 90.3998) (width 0.3) (layer B.Cu) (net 6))
 (segment (start 141.2 106) (end 141.2 106.6601) (width 0.3) (layer B.Cu) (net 6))
 (segment (start 141.2 106.6601) (end 141.1999 106.6601) (width 0.3) (layer B.Cu) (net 6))
 (segment (start 141.1999 106.6601) (end 141.1999 107.4) (width 0.3) (layer B.Cu) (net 6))
 (segment (start 142.8001 107.4001) (end 142.8001 107.4) (width 0.3) (layer B.Cu) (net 14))
 (segment (start 142.9 108.95) (end 142.9 107.5) (width 0.3) (layer B.Cu) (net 14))
 (segment (start 142.9 107.5) (end 142.8001 107.4001) (width 0.3) (layer B.Cu) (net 14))
 (segment (start 142.8001 107.4001) (end 142.8 107.4) (width 0.3) (layer B.Cu) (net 14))
 (segment (start 142.8 107.4) (end 142.8 106.1) (width 0.3) (layer B.Cu) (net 14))
 (segment (start 142.8 105.2) (end 142.8 102.3) (width 0.3) (layer B.Cu) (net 11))
 (segment (start 151.3 81.7) (end 151.3 78.3002) (width 0.6) (layer B.Cu) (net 3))
 (segment (start 146 85.4302) (end 150.07 85.4302) (width 0.6) (layer B.Cu) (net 3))
 (segment (start 150.07 85.4302) (end 151.3 84.2) (width 0.6) (layer B.Cu) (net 3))
 (segment (start 151.3 84.2) (end 151.3 81.7) (width 0.6) (layer B.Cu) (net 3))
 (segment (start 147.2 81.7) (end 149 81.7) (width 0.6) (layer B.Cu) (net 3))
 (segment (start 145.574 81.7) (end 147.2 81.7) (width 0.6) (layer B.Cu) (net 3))
 (segment (start 144.2 90.3998) (end 144.2 88.9) (width 0.6) (layer B.Cu) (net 3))
 (segment (start 144.2 88.9) (end 145.3 88.9) (width 0.6) (layer B.Cu) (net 3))
 (segment (start 145.3 88.9) (end 146 88.2) (width 0.6) (layer B.Cu) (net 3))
 (segment (start 146 88.2) (end 146 85.4302) (width 0.6) (layer B.Cu) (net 3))
 (segment (start 145.574 83.6) (end 145.574 85.004) (width 0.3) (layer B.Cu) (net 3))
 (segment (start 145.574 85.004) (end 146 85.4302) (width 0.3) (layer B.Cu) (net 3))
 (segment (start 149 81.7) (end 151.3 81.7) (width 0.6) (layer B.Cu) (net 3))
 (segment (start 142.8 96.4) (end 142.8 96.36) (width 0.3) (layer B.Cu) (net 10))
 (segment (start 142.8 99.4) (end 142.8 96.4) (width 0.3) (layer B.Cu) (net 10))
 (segment (start 141.9 96.4) (end 138.9 96.4) (width 0.3) (layer B.Cu) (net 21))
 (segment (start 138.9 96.4) (end 137.8 96.4) (width 0.3) (layer B.Cu) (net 21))
 (segment (start 140.5 92) (end 138.95 92) (width 0.3) (layer B.Cu) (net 13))
 (segment (start 140.5 92) (end 141.9 92) (width 0.3) (layer B.Cu) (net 13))
 (segment (start 142.8 92) (end 144.2 92) (width 0.3) (layer B.Cu) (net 7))
 (segment (start 144.2 92) (end 150 92) (width 0.3) (layer B.Cu) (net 7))
 (segment (start 148.7 76.13) (end 148.7001 76.1301) (width 0.3) (layer B.Cu) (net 16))
 (segment (start 148.7001 76.1301) (end 148.7001 76.7) (width 0.3) (layer B.Cu) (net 16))
 (segment (start 148.7 76.13) (end 148.7 76.7) (width 0.4) (layer B.Cu) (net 16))
 (segment (start 148.7 74.525) (end 148.7 76.13) (width 0.4) (layer B.Cu) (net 16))
 (segment (start 151.3 74.525) (end 151.3 76.7) (width 0.4) (layer B.Cu) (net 15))
 (segment (start 145.1 110.25) (end 149.75 110.25) (width 0.3) (layer B.Cu) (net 23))
 (segment (start 149.75 110.25) (end 150 110) (width 0.3) (layer B.Cu) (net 23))
 (segment (start 150 110) (end 150 109) (width 0.3) (layer B.Cu) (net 23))
 (segment (start 137.65 94.2) (end 137.65 95.29) (width 0.3) (layer B.Cu) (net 24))
 (segment (start 137.65 95.29) (end 137.8 95.44) (width 0.3) (layer B.Cu) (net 24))
 (segment (start 149.04 105.2) (end 143.76 105.2) (width 0.3) (layer B.Cu) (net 1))
 (segment (start 142.9 110.25) (end 141.55 110.25) (width 0.4) (layer B.Cu) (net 12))
 (segment (start 141.55 110.25) (end 141.2 110.6) (width 0.4) (layer B.Cu) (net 12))
 (segment (start 142.8 95.4) (end 142.8 92.96) (width 0.3) (layer B.Cu) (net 8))
 (segment (start 137.65 92) (end 137.65 90.75) (width 0.4) (layer B.Cu) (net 9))
 (segment (start 137.65 90.75) (end 137.3 90.4) (width 0.4) (layer B.Cu) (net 9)))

